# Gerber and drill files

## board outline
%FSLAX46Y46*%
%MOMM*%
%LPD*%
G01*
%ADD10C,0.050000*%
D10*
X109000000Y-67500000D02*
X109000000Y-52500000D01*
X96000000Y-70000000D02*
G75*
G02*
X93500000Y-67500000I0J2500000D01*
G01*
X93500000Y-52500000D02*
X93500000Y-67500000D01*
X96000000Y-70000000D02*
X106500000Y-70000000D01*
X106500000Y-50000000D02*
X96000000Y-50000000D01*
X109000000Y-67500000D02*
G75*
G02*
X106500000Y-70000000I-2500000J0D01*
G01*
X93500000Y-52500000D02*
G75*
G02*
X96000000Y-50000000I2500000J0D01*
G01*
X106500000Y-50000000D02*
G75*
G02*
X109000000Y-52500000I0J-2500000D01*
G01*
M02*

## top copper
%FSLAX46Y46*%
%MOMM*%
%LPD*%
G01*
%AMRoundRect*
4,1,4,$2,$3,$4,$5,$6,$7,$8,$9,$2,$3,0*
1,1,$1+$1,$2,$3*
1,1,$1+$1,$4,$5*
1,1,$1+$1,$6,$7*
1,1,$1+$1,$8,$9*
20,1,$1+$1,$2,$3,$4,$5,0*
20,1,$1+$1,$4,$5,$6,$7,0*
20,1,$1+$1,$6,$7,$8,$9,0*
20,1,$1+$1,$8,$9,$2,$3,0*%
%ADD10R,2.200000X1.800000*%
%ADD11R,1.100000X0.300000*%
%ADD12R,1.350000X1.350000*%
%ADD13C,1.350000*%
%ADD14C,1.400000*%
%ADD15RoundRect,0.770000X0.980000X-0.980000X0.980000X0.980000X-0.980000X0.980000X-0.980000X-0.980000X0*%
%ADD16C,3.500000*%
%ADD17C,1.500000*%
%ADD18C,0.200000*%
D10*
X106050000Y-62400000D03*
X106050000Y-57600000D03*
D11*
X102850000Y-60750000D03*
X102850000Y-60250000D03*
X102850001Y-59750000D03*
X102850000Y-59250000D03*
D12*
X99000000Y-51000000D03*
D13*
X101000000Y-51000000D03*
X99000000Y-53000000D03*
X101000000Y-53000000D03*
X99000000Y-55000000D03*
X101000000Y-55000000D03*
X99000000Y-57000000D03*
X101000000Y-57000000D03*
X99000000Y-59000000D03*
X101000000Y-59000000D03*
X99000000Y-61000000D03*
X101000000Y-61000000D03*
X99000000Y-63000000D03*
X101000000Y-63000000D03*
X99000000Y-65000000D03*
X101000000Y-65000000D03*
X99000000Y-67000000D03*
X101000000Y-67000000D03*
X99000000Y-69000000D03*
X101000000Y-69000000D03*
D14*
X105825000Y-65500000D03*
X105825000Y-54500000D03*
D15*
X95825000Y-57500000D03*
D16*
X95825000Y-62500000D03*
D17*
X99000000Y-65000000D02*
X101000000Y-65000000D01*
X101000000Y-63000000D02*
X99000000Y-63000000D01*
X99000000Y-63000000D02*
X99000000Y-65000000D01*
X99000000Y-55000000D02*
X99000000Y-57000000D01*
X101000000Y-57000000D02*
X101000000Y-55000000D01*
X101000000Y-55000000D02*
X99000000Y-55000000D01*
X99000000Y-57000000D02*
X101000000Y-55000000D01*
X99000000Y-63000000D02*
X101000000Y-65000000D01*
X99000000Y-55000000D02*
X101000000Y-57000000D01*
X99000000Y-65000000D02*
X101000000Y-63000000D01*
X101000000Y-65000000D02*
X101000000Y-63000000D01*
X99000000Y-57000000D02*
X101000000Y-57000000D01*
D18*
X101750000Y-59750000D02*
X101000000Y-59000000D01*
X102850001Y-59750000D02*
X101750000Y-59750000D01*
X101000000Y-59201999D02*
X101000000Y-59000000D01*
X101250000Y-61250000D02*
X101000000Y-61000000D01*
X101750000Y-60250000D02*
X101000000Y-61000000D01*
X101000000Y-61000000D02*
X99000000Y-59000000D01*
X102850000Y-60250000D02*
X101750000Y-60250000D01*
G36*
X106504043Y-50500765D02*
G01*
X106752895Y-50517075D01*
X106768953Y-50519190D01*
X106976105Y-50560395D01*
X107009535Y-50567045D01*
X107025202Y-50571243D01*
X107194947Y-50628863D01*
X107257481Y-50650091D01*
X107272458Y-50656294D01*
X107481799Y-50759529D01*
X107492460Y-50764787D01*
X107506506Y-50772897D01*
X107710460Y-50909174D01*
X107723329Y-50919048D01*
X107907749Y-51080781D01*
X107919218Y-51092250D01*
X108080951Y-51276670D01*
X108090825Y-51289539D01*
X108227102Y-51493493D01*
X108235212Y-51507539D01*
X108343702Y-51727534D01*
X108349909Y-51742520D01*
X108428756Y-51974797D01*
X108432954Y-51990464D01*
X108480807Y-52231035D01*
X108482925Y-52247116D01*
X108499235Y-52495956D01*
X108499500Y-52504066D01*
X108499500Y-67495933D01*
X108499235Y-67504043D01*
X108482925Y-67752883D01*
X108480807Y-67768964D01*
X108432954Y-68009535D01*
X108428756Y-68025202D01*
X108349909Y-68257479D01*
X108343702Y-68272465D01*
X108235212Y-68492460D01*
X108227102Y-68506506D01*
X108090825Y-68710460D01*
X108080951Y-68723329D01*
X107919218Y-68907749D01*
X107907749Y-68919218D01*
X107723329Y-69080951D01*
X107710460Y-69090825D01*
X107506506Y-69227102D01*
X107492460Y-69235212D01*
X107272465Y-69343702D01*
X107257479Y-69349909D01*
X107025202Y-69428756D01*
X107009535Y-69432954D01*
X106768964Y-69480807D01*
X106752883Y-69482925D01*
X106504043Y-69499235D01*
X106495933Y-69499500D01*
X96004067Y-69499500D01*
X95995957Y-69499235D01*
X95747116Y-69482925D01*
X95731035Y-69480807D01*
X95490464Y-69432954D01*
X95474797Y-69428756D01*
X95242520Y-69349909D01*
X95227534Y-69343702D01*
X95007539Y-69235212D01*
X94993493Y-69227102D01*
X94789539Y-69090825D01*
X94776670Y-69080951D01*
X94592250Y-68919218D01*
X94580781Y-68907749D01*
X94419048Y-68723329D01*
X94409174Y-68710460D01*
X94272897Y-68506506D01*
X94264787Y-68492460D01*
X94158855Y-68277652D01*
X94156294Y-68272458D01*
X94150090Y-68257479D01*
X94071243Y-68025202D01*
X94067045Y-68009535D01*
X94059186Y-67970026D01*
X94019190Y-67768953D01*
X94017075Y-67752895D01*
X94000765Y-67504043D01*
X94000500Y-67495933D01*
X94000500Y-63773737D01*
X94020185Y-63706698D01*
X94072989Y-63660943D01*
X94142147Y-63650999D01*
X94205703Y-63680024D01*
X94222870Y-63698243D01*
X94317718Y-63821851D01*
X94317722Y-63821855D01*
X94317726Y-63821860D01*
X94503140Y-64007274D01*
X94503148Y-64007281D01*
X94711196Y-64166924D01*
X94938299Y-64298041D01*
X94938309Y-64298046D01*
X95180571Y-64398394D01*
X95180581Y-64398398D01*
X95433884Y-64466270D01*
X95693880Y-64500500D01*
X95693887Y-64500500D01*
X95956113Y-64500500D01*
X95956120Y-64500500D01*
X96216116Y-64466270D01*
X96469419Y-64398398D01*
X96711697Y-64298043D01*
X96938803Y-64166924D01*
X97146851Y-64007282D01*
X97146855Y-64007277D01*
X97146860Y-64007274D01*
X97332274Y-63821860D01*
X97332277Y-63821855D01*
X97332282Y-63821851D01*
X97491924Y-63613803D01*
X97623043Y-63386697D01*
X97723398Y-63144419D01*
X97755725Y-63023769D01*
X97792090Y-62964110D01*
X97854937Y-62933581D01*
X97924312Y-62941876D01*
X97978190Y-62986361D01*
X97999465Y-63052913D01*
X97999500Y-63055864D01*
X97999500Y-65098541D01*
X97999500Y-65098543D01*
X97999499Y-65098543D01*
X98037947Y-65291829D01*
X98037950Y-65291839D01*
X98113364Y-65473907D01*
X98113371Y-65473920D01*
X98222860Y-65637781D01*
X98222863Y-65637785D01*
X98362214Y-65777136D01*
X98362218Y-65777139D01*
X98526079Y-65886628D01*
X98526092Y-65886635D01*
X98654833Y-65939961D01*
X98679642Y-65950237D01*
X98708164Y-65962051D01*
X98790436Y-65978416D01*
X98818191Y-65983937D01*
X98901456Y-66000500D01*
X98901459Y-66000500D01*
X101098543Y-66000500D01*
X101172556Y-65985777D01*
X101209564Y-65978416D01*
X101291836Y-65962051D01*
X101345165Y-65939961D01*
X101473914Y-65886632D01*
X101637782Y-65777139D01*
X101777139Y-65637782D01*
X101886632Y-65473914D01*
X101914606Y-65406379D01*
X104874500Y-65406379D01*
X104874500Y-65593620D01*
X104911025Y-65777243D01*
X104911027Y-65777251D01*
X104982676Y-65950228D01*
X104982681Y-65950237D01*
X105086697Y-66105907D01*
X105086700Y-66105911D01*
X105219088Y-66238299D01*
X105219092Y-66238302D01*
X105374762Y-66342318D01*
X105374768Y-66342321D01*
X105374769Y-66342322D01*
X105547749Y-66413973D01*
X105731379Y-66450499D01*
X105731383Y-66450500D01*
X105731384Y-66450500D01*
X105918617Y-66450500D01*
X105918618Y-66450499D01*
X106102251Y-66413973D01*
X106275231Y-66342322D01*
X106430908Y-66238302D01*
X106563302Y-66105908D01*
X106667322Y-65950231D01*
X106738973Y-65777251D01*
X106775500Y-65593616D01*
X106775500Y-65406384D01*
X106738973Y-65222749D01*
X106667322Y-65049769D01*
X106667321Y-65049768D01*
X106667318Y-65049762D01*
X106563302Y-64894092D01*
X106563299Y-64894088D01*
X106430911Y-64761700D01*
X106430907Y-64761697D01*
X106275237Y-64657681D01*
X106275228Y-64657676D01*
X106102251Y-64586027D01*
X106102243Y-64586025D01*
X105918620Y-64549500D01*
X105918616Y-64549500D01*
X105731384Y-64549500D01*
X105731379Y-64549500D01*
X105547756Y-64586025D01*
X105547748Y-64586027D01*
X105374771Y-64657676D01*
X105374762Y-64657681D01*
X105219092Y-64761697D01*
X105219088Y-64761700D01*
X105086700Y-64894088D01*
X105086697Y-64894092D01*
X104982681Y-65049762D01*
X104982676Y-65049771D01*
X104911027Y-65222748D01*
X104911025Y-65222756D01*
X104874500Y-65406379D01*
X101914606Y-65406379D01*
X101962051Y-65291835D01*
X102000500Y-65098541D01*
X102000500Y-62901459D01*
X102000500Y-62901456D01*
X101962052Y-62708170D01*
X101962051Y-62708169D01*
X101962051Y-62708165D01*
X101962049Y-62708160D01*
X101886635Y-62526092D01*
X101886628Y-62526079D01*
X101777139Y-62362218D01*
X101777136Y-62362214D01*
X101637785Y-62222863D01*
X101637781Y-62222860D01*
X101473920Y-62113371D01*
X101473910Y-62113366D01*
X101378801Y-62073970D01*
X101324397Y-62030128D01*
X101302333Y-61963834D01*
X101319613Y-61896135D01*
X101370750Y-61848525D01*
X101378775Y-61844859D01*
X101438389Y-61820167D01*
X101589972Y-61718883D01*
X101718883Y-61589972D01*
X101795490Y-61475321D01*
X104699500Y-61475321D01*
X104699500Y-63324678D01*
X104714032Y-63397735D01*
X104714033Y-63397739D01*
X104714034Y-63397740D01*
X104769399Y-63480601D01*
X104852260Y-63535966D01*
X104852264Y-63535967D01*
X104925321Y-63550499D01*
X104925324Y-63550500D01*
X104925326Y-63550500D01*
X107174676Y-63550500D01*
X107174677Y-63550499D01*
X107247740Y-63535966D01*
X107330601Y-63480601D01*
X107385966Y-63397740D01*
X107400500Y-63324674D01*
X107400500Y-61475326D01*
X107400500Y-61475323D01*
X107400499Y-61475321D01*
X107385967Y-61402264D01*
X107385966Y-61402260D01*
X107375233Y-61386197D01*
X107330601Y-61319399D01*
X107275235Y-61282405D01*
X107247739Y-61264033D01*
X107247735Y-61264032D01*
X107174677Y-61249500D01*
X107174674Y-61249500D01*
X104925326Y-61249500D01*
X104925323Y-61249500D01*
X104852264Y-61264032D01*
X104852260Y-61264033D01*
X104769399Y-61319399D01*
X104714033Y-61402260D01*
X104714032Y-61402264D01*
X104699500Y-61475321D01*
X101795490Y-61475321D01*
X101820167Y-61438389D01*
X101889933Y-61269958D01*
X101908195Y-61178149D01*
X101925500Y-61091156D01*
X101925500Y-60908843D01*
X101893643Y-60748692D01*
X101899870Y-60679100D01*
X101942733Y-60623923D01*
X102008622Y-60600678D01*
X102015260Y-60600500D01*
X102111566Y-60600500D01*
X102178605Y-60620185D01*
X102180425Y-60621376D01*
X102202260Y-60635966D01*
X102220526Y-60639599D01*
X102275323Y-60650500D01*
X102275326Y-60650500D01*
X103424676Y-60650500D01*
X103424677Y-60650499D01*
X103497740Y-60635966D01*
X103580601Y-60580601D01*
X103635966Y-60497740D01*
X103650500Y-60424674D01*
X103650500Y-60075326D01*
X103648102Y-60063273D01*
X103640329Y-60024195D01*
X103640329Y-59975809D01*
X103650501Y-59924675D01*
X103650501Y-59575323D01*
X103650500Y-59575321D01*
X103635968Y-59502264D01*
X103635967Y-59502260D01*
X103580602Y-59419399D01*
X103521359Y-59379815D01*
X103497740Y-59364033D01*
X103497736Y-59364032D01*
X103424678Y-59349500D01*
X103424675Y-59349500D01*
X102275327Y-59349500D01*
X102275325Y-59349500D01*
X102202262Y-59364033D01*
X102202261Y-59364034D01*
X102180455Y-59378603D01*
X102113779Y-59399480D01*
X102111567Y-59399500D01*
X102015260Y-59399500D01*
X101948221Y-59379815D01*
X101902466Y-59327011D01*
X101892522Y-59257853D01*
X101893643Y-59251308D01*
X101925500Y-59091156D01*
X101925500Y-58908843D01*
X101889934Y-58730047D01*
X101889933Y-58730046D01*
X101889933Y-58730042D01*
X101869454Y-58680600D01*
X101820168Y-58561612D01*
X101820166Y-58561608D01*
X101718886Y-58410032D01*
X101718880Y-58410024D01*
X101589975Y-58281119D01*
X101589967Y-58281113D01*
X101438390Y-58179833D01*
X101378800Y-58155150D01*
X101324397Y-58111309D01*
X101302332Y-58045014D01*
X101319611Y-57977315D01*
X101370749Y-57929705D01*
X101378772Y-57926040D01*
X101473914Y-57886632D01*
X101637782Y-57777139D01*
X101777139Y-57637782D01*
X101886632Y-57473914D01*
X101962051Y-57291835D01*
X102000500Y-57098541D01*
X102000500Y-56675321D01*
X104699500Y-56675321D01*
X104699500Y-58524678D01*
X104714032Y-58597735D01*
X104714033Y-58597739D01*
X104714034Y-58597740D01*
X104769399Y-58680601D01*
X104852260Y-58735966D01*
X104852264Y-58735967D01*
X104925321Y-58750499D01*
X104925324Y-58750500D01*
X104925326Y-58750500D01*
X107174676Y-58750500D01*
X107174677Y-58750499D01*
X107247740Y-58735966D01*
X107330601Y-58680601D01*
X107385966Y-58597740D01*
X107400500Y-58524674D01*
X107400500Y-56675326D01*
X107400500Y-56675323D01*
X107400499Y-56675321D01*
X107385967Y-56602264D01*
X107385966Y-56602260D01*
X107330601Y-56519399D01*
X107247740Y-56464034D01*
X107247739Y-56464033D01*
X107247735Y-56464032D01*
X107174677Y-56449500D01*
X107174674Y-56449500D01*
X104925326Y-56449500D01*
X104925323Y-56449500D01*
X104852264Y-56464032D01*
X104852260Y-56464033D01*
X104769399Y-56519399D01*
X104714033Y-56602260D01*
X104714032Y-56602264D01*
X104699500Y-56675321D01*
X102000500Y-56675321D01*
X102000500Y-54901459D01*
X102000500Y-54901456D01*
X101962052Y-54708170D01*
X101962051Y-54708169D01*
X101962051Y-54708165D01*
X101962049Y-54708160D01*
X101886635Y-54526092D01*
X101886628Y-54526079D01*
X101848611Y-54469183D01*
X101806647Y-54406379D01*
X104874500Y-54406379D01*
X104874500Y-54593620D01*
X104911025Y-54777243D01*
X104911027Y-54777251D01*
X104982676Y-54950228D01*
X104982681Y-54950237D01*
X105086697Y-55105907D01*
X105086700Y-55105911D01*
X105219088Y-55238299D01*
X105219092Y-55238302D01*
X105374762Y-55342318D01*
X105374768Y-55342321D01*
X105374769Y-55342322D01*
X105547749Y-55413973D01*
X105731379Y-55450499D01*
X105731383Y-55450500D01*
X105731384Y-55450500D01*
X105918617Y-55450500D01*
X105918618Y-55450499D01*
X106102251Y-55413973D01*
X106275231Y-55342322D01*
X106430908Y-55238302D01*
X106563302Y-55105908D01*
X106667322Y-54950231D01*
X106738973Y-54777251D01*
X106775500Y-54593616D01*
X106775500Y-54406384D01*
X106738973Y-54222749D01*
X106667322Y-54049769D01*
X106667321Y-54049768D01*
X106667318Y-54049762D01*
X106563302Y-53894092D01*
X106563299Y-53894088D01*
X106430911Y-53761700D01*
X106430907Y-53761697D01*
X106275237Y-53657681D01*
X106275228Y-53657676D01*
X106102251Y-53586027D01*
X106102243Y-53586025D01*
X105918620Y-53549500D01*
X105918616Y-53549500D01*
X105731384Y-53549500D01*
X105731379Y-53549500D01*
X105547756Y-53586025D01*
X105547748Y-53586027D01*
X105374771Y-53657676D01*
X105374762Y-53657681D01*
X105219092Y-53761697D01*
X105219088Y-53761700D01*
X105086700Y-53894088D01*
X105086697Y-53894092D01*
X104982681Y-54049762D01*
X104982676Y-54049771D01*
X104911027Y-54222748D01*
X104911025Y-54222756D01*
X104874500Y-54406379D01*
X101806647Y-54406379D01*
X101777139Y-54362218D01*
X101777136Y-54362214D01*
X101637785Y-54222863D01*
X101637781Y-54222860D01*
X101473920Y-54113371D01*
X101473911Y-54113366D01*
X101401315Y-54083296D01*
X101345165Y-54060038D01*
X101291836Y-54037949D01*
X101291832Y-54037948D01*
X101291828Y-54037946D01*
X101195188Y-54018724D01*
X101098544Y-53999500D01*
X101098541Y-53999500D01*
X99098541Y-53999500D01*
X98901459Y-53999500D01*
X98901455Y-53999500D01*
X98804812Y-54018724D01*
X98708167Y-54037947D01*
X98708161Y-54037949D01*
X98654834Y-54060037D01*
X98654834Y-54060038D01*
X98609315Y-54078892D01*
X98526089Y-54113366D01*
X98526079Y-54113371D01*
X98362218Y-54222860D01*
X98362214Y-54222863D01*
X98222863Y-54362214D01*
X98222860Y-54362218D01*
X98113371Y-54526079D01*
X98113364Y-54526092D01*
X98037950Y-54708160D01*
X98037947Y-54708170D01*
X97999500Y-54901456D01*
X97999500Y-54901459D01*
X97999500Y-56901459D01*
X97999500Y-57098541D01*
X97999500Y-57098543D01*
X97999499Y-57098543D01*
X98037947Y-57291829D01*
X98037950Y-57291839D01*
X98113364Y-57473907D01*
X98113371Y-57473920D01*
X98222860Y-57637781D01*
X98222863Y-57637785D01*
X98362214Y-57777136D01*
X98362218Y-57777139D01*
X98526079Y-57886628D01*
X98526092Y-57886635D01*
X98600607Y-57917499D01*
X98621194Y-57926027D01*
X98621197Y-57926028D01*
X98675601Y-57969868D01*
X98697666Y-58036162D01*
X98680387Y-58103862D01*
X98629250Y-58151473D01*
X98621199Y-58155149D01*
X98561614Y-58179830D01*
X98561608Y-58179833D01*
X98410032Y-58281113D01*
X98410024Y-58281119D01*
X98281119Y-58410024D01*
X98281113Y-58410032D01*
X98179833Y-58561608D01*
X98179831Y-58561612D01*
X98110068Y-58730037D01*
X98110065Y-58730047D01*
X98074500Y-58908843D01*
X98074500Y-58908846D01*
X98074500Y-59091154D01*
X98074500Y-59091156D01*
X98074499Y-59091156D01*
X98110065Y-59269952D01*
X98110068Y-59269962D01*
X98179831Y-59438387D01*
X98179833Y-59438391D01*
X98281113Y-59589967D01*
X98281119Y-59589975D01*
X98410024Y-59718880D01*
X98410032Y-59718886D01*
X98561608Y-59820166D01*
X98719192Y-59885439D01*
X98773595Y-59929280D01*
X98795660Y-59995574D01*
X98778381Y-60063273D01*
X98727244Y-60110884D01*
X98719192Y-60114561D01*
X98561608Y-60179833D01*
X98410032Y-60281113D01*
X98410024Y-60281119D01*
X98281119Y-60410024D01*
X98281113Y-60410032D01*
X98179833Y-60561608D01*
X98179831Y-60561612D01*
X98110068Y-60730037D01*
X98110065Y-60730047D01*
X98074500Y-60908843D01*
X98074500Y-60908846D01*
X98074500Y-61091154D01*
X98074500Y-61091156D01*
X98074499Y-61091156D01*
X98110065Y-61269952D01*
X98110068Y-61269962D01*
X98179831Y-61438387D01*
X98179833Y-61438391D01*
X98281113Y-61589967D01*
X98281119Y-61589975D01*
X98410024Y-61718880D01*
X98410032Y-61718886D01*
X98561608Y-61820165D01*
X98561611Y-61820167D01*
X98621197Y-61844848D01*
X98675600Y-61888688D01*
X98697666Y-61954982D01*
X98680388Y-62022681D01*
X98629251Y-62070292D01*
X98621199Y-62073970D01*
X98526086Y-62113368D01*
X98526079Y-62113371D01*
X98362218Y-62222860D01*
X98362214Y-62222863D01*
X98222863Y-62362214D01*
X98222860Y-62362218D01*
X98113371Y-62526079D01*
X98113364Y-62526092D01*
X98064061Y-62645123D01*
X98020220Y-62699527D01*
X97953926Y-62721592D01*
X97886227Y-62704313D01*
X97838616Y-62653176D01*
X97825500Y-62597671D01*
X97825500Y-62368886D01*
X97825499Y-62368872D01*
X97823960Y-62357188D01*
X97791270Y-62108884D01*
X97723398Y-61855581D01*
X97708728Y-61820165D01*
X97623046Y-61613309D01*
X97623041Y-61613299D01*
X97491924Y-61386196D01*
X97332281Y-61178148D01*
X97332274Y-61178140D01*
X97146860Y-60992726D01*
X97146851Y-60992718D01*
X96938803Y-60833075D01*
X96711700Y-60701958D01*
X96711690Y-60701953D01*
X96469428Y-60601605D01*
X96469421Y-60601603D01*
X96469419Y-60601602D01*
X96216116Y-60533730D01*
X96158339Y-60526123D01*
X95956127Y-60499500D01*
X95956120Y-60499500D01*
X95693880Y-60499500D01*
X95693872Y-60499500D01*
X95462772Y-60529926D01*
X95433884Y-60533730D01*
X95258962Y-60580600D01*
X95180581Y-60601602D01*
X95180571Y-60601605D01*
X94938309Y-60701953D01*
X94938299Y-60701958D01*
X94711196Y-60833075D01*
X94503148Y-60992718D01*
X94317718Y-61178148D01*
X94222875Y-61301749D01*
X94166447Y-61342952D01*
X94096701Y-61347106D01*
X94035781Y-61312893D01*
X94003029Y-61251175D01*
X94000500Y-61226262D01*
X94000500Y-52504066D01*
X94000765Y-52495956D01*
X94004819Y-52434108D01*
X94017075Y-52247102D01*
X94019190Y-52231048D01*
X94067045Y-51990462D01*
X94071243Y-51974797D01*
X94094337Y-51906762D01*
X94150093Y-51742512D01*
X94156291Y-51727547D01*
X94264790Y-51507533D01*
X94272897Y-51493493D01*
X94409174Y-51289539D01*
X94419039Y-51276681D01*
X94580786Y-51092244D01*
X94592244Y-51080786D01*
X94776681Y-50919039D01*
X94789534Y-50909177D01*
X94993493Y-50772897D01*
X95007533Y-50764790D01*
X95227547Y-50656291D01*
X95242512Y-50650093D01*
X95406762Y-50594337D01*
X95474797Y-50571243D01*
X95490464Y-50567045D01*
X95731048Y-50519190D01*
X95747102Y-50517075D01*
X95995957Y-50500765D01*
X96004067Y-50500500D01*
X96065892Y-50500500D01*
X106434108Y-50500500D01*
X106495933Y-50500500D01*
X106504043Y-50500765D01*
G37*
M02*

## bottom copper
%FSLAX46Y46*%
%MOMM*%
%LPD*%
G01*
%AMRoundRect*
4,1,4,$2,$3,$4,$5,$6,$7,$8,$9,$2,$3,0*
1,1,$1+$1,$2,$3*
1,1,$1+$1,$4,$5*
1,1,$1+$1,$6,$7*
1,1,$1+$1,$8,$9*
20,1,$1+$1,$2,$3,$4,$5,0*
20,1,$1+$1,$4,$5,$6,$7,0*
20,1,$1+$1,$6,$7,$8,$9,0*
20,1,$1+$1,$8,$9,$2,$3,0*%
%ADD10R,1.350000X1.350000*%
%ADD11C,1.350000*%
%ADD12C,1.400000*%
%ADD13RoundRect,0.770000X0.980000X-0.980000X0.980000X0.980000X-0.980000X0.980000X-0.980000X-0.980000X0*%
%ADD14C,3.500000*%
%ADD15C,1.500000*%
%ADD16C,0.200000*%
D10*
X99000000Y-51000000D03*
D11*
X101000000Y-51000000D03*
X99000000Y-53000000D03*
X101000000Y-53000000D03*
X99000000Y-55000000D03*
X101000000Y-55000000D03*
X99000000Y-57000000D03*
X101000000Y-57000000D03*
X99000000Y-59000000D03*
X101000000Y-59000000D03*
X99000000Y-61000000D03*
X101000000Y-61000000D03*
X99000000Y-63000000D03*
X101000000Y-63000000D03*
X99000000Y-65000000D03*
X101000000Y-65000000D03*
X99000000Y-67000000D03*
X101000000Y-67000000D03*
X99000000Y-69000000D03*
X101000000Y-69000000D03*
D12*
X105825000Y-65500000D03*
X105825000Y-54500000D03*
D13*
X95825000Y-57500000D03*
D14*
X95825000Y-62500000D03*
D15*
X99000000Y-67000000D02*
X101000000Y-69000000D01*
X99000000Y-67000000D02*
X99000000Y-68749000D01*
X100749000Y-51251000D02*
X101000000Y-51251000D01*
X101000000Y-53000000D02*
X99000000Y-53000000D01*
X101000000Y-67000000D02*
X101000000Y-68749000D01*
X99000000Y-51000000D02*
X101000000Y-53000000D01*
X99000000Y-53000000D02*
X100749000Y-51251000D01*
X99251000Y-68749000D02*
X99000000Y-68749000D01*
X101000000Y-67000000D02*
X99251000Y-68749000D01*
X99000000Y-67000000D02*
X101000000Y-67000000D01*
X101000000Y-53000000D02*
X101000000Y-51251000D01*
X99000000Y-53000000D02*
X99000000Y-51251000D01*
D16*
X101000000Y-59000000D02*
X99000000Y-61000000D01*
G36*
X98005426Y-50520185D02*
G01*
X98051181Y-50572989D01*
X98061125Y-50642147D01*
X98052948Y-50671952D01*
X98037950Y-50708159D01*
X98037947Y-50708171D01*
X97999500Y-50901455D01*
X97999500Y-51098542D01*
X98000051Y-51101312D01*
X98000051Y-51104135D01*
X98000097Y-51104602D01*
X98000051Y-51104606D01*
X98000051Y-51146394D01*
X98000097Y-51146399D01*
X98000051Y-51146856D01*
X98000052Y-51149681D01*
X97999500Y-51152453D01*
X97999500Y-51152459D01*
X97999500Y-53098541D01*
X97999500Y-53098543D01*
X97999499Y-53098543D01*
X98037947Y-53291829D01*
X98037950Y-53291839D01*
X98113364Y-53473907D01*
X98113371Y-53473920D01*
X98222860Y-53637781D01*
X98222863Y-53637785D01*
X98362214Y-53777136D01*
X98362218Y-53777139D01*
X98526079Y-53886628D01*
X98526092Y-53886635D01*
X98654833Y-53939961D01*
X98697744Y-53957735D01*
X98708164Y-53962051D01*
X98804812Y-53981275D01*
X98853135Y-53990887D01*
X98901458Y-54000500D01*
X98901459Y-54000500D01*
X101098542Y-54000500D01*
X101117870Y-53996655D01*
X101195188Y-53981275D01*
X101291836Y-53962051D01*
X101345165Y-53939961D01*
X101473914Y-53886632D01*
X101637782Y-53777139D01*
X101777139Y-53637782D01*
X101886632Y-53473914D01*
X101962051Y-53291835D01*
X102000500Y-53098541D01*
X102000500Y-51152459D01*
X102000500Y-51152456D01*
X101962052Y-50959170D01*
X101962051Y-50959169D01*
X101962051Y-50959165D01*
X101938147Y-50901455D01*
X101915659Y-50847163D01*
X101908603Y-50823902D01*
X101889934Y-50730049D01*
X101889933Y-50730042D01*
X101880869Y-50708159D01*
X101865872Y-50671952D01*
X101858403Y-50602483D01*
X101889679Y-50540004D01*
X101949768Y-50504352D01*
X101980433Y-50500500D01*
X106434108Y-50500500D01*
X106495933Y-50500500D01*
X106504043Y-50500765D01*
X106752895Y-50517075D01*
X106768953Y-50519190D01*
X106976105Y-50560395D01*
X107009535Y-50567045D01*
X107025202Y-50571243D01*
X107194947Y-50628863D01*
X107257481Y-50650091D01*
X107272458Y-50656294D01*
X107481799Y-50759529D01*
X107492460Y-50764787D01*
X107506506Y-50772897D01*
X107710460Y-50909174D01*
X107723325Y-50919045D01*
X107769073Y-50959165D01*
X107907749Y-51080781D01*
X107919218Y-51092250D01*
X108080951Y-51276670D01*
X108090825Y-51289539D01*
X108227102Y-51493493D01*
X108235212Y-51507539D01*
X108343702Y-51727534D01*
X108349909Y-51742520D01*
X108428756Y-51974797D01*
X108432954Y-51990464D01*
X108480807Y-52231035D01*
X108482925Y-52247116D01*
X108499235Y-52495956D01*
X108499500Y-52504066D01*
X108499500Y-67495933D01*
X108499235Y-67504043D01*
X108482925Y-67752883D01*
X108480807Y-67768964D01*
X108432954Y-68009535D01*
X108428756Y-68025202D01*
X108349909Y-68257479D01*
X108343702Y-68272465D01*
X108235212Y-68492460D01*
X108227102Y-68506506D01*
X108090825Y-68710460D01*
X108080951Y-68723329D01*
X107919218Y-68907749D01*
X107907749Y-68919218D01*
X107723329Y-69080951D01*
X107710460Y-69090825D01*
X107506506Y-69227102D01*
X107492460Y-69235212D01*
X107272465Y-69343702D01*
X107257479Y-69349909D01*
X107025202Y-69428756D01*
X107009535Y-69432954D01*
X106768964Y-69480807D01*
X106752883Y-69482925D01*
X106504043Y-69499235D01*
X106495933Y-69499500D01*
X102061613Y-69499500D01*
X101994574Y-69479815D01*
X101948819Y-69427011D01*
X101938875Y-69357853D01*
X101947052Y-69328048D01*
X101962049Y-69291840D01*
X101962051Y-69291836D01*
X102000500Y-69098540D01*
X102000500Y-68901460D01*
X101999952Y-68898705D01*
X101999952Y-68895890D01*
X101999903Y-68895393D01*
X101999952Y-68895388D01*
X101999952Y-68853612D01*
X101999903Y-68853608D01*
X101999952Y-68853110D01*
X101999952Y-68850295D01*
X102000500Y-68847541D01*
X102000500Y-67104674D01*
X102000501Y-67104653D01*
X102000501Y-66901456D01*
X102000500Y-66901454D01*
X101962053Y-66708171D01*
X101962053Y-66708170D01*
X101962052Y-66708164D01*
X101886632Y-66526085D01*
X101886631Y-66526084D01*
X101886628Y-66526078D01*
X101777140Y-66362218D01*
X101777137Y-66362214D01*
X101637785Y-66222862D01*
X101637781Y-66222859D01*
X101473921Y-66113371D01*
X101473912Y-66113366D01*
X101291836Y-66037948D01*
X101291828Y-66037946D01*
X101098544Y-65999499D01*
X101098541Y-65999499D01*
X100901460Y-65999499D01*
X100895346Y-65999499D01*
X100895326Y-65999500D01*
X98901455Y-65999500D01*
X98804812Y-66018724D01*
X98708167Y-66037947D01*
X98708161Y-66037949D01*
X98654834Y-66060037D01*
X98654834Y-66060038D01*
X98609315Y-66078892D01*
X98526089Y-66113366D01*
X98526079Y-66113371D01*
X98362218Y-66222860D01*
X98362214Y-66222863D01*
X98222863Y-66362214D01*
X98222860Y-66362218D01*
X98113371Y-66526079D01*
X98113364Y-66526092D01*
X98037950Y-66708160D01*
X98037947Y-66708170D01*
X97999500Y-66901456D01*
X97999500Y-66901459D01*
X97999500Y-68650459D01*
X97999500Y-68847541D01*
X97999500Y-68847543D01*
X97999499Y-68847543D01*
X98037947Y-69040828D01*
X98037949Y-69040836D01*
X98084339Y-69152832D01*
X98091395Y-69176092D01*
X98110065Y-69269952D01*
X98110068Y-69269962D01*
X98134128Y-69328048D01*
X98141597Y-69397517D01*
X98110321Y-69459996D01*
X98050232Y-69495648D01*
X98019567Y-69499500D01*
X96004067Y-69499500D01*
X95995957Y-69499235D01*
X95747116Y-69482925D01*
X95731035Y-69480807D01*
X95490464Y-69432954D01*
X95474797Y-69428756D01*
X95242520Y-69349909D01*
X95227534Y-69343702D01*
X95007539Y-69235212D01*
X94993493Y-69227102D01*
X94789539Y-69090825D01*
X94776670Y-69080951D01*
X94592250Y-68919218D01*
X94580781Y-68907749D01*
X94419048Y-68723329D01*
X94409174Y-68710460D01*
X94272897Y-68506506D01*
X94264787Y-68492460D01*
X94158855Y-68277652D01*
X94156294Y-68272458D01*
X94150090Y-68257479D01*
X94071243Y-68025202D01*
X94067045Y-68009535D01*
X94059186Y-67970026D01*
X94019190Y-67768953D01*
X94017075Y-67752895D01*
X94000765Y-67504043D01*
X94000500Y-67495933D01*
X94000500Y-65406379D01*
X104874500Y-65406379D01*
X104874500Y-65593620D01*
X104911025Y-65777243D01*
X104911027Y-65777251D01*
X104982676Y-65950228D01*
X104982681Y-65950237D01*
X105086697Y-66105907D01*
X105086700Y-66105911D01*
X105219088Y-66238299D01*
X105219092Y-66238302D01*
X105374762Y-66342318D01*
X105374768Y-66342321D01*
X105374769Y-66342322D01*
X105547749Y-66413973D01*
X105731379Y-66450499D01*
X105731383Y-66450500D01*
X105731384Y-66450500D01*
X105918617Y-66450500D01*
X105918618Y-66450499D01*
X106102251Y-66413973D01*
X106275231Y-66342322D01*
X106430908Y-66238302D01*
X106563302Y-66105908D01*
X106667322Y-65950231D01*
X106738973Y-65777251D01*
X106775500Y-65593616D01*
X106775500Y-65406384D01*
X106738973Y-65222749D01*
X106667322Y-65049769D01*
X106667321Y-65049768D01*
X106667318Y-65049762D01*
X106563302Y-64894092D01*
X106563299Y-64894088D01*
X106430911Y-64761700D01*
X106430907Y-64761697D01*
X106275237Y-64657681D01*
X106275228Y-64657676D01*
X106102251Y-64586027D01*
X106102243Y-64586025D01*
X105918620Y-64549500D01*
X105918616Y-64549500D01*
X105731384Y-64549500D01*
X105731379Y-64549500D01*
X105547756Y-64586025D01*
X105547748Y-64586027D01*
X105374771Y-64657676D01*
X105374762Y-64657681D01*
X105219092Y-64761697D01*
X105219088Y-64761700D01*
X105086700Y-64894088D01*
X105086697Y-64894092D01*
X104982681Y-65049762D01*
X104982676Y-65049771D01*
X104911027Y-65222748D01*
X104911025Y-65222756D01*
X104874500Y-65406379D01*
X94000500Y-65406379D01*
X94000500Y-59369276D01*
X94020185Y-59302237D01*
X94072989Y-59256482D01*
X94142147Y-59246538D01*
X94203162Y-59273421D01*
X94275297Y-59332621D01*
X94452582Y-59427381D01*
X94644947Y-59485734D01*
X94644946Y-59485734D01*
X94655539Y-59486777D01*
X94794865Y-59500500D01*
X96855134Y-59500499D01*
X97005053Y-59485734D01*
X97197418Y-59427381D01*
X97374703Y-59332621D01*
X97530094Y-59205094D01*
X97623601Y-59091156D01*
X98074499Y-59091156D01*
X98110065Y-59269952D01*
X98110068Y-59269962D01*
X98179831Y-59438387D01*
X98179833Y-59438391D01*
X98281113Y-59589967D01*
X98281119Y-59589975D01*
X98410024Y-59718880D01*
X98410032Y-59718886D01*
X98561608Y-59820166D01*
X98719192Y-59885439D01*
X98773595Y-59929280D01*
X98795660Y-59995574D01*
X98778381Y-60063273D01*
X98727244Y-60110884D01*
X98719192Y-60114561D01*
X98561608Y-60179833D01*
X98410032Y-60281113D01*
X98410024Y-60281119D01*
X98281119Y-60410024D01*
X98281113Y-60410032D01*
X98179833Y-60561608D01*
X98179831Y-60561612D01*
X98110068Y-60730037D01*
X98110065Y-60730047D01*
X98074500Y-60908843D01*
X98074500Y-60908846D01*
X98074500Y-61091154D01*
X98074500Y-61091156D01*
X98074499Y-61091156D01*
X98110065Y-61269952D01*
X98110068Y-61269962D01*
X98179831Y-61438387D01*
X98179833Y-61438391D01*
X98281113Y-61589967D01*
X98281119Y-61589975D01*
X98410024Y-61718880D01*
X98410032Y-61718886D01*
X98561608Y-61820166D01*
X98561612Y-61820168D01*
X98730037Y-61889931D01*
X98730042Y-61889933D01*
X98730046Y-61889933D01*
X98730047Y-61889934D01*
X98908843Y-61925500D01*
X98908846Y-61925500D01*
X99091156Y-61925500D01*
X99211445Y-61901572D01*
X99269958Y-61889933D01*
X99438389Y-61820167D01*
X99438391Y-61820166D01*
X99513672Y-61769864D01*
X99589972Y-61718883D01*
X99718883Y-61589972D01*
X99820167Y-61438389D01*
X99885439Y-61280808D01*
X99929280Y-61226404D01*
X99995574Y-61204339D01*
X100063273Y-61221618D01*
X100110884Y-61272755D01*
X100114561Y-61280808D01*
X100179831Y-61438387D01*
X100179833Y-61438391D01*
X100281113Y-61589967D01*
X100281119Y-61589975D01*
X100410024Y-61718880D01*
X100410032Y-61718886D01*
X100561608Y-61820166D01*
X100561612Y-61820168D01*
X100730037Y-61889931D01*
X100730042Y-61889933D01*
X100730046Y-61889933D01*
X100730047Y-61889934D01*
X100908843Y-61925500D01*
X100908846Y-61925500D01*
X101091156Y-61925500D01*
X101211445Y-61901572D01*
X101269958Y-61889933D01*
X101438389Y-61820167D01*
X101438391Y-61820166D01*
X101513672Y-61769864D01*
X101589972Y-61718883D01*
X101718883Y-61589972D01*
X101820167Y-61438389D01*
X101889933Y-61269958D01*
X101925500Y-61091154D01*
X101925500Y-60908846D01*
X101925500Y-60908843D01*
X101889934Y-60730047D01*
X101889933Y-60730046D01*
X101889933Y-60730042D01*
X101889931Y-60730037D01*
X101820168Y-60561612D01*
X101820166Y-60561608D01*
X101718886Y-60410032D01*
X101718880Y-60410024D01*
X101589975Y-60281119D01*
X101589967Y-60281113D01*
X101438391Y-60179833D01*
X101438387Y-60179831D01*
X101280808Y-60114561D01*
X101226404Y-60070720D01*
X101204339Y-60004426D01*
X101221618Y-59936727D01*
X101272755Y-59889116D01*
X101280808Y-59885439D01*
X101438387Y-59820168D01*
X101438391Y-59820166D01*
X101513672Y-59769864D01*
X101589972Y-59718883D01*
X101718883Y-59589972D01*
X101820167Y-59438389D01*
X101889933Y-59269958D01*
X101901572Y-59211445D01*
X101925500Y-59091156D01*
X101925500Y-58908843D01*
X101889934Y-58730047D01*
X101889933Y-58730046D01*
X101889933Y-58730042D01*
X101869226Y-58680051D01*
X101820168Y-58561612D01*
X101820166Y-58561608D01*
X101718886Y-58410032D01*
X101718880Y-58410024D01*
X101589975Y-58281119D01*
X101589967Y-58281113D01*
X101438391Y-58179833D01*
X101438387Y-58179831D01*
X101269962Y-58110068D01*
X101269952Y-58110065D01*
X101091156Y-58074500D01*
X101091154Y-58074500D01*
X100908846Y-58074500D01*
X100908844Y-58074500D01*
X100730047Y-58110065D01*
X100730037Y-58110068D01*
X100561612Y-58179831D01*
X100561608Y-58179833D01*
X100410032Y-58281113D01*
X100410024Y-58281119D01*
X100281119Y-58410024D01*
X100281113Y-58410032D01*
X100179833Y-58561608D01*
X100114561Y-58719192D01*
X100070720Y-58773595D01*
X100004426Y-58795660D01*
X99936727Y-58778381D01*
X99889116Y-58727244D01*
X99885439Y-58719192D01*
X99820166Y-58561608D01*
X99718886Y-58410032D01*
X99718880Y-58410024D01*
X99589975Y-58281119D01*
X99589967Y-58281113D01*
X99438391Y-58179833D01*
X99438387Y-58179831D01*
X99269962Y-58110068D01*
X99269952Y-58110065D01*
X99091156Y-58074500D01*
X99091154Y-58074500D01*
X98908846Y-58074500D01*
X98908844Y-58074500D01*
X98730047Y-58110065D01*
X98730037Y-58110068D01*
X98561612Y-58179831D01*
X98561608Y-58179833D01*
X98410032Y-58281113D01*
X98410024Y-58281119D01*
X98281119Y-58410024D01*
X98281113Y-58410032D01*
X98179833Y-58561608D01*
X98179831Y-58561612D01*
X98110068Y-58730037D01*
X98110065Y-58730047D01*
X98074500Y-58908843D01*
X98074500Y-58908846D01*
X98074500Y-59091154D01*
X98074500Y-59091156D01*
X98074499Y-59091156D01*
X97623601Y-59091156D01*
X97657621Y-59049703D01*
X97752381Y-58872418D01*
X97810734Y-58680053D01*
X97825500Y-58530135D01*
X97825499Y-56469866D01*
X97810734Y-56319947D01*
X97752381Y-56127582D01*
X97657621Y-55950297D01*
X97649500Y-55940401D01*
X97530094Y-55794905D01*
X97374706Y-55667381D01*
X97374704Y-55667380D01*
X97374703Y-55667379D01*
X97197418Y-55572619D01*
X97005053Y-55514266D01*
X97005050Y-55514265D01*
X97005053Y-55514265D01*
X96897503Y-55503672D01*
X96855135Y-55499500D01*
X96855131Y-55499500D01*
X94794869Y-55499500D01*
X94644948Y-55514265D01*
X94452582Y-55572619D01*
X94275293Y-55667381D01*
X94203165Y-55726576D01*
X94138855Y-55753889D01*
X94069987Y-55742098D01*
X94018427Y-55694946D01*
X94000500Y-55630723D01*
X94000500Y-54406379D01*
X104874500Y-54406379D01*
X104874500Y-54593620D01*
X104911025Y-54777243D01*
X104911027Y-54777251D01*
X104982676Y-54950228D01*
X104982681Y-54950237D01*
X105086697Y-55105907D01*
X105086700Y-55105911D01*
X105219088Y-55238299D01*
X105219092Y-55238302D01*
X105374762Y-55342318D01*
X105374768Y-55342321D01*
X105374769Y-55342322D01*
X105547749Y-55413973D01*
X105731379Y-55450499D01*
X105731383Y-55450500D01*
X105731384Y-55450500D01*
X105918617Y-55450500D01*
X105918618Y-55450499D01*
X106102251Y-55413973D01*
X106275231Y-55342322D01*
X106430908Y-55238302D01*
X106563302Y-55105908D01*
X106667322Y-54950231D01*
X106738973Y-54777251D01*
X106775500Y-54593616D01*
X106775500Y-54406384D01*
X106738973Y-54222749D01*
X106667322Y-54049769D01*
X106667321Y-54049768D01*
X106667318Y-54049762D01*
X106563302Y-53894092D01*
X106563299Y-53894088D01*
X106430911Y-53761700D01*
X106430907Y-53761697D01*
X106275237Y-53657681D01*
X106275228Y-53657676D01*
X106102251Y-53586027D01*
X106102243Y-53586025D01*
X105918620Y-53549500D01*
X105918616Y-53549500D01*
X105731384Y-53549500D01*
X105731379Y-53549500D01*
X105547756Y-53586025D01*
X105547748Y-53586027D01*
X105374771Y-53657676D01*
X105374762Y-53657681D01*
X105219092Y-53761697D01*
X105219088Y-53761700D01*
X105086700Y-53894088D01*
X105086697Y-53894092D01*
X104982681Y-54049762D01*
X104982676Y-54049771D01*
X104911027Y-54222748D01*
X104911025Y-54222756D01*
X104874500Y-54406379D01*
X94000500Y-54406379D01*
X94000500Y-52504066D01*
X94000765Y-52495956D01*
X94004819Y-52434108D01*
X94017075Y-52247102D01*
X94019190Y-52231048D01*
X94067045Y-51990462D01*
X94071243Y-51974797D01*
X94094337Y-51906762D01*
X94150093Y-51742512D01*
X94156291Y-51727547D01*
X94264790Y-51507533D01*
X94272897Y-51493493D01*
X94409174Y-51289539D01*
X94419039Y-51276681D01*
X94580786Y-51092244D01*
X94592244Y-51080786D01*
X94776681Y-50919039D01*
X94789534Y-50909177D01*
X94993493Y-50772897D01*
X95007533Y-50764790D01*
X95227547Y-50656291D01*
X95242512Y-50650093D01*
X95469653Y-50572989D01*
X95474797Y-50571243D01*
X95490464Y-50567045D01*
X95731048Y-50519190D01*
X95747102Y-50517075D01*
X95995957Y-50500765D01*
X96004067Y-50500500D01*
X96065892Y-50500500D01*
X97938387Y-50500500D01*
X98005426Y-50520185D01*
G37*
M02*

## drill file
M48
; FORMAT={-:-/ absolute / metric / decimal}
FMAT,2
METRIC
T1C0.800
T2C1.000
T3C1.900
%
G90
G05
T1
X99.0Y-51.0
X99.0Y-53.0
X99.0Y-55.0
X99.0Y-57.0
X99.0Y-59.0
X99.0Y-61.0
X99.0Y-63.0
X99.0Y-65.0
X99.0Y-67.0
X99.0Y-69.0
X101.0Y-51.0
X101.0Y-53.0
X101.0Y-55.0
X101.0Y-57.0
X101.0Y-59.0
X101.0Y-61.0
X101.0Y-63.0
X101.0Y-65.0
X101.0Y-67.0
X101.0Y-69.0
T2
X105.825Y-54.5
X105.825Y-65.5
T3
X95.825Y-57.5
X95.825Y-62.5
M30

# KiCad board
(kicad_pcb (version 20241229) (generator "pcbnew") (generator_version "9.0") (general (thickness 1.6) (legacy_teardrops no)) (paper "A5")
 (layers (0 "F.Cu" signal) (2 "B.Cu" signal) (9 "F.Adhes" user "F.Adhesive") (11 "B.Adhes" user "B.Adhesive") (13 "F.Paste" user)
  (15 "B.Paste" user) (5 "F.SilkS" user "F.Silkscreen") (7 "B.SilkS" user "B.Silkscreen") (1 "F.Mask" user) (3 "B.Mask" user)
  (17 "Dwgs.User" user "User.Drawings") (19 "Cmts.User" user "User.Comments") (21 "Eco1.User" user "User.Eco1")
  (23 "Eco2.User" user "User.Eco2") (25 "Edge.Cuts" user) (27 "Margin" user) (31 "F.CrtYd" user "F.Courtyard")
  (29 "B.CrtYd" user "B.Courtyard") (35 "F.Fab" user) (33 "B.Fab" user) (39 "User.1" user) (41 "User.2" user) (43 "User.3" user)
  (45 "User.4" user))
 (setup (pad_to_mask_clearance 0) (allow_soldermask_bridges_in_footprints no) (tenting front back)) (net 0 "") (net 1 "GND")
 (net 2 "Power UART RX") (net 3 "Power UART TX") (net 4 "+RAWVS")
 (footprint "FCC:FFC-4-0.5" (layer "F.Cu") (at 103.5 60 90)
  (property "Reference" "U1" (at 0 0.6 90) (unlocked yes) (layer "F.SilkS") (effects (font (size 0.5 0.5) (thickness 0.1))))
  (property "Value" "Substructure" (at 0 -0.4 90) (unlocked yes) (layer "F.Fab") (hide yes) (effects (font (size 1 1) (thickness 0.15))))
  (pad "" smd rect (at -2.4 2.55 90) (size 1.8 2.2) (layers "F.Cu" "F.Mask" "F.Paste") (thermal_bridge_angle 45))
  (pad "" smd rect (at 2.4 2.55 90) (size 1.8 2.2) (layers "F.Cu" "F.Mask" "F.Paste") (thermal_bridge_angle 45))
  (pad "1" smd rect (at -0.75 -0.65 90) (size 0.3 1.1) (layers "F.Cu" "F.Mask" "F.Paste") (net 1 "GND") (thermal_bridge_angle 45))
  (pad "2" smd rect (at -0.25 -0.65 90) (size 0.3 1.1) (layers "F.Cu" "F.Mask" "F.Paste") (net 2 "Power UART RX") (thermal_bridge_angle 45))
  (pad "3" smd rect (at 0.25 -0.649999 90) (size 0.3 1.1) (layers "F.Cu" "F.Mask" "F.Paste") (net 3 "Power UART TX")
   (thermal_bridge_angle 45))
  (pad "4" smd rect (at 0.75 -0.65 90) (size 0.3 1.1) (layers "F.Cu" "F.Mask" "F.Paste") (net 1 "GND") (thermal_bridge_angle 45)))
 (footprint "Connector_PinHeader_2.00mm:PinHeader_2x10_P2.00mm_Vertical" (layer "F.Cu") (at 99 51)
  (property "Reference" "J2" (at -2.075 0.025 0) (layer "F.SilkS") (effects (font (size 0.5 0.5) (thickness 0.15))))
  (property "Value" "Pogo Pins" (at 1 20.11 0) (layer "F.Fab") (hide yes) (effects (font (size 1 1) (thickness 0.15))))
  (pad "1" thru_hole rect (at 0 0) (size 1.35 1.35) (drill 0.8) (layers "*.Cu" "*.Mask") (remove_unused_layers no) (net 1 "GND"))
  (pad "2" thru_hole circle (at 2 0) (size 1.35 1.35) (drill 0.8) (layers "*.Cu" "*.Mask") (remove_unused_layers no) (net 1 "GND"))
  (pad "3" thru_hole circle (at 0 2) (size 1.35 1.35) (drill 0.8) (layers "*.Cu" "*.Mask") (remove_unused_layers no) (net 1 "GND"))
  (pad "4" thru_hole circle (at 2 2) (size 1.35 1.35) (drill 0.8) (layers "*.Cu" "*.Mask") (remove_unused_layers no) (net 1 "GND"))
  (pad "5" thru_hole circle (at 0 4) (size 1.35 1.35) (drill 0.8) (layers "*.Cu" "*.Mask") (remove_unused_layers no) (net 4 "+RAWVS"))
  (pad "6" thru_hole circle (at 2 4) (size 1.35 1.35) (drill 0.8) (layers "*.Cu" "*.Mask") (remove_unused_layers no) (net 4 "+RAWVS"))
  (pad "7" thru_hole circle (at 0 6) (size 1.35 1.35) (drill 0.8) (layers "*.Cu" "*.Mask") (remove_unused_layers no) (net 4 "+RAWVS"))
  (pad "8" thru_hole circle (at 2 6) (size 1.35 1.35) (drill 0.8) (layers "*.Cu" "*.Mask") (remove_unused_layers no) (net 4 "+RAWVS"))
  (pad "9" thru_hole circle (at 0 8) (size 1.35 1.35) (drill 0.8) (layers "*.Cu" "*.Mask") (remove_unused_layers no) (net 2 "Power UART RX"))
  (pad "10" thru_hole circle (at 2 8) (size 1.35 1.35) (drill 0.8) (layers "*.Cu" "*.Mask") (remove_unused_layers no)
   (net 3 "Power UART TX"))
  (pad "11" thru_hole circle (at 0 10) (size 1.35 1.35) (drill 0.8) (layers "*.Cu" "*.Mask") (remove_unused_layers no)
   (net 3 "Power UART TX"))
  (pad "12" thru_hole circle (at 2 10) (size 1.35 1.35) (drill 0.8) (layers "*.Cu" "*.Mask") (remove_unused_layers no)
   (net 2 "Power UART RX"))
  (pad "13" thru_hole circle (at 0 12) (size 1.35 1.35) (drill 0.8) (layers "*.Cu" "*.Mask") (remove_unused_layers no) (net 4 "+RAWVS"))
  (pad "14" thru_hole circle (at 2 12) (size 1.35 1.35) (drill 0.8) (layers "*.Cu" "*.Mask") (remove_unused_layers no) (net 4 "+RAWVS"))
  (pad "15" thru_hole circle (at 0 14) (size 1.35 1.35) (drill 0.8) (layers "*.Cu" "*.Mask") (remove_unused_layers no) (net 4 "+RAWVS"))
  (pad "16" thru_hole circle (at 2 14) (size 1.35 1.35) (drill 0.8) (layers "*.Cu" "*.Mask") (remove_unused_layers no) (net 4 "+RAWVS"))
  (pad "17" thru_hole circle (at 0 16) (size 1.35 1.35) (drill 0.8) (layers "*.Cu" "*.Mask") (remove_unused_layers no) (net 1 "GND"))
  (pad "18" thru_hole circle (at 2 16) (size 1.35 1.35) (drill 0.8) (layers "*.Cu" "*.Mask") (remove_unused_layers no) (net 1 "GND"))
  (pad "19" thru_hole circle (at 0 18) (size 1.35 1.35) (drill 0.8) (layers "*.Cu" "*.Mask") (remove_unused_layers no) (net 1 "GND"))
  (pad "20" thru_hole circle (at 2 18) (size 1.35 1.35) (drill 0.8) (layers "*.Cu" "*.Mask") (remove_unused_layers no) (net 1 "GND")))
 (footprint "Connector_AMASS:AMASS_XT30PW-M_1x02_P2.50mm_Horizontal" (layer "B.Cu") (at 95.825 57.5 90)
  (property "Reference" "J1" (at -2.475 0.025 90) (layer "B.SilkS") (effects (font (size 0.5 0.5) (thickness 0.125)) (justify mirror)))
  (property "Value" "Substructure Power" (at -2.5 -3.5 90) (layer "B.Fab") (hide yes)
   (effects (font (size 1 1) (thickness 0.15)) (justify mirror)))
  (pad "" thru_hole circle (at -8 10 90) (size 1.4 1.4) (drill 1) (layers "*.Cu" "*.Mask") (remove_unused_layers no))
  (pad "" thru_hole circle (at 3 10 90) (size 1.4 1.4) (drill 1) (layers "*.Cu" "*.Mask") (remove_unused_layers no))
  (pad "1" thru_hole roundrect (at 0 0 90) (size 3.5 3.5) (drill 1.9) (layers "*.Cu" "*.Mask") (remove_unused_layers no)
   (roundrect_rratio 0.22) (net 1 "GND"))
  (pad "2" thru_hole circle (at -5 0 90) (size 3.5 3.5) (drill 1.9) (layers "*.Cu" "*.Mask") (remove_unused_layers no) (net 4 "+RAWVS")))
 (gr_line (start 109 67.5) (end 109 52.5) (stroke (width 0.05) (type default)) (layer "Edge.Cuts"))
 (gr_arc (start 96 70) (mid 94.232233 69.267767) (end 93.5 67.5) (stroke (width 0.05) (type default)) (layer "Edge.Cuts"))
 (gr_line (start 93.5 52.5) (end 93.5 67.5) (stroke (width 0.05) (type default)) (layer "Edge.Cuts"))
 (gr_line (start 96 70) (end 106.5 70) (stroke (width 0.05) (type default)) (layer "Edge.Cuts"))
 (gr_line (start 106.5 50) (end 96 50) (stroke (width 0.05) (type default)) (layer "Edge.Cuts"))
 (gr_arc (start 109 67.5) (mid 108.267767 69.267767) (end 106.5 70) (stroke (width 0.05) (type default)) (layer "Edge.Cuts"))
 (gr_arc (start 93.5 52.5) (mid 94.232233 50.732233) (end 96 50) (stroke (width 0.05) (type default)) (layer "Edge.Cuts"))
 (gr_arc (start 106.5 50) (mid 108.267767 50.732233) (end 109 52.5) (stroke (width 0.05) (type default)) (layer "Edge.Cuts"))
 (segment (start 99 65) (end 101 65) (width 1.5) (layer "F.Cu") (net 4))
 (segment (start 101 63) (end 99 63) (width 1.5) (layer "F.Cu") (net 4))
 (segment (start 99 63) (end 99 65) (width 1.5) (layer "F.Cu") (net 4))
 (segment (start 99 55) (end 99 57) (width 1.5) (layer "F.Cu") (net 4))
 (segment (start 101 57) (end 101 55) (width 1.5) (layer "F.Cu") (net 4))
 (segment (start 101 55) (end 99 55) (width 1.5) (layer "F.Cu") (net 4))
 (segment (start 99 57) (end 101 55) (width 1.5) (layer "F.Cu") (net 4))
 (segment (start 99 63) (end 101 65) (width 1.5) (layer "F.Cu") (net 4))
 (segment (start 99 55) (end 101 57) (width 1.5) (layer "F.Cu") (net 4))
 (segment (start 99 65) (end 101 63) (width 1.5) (layer "F.Cu") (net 4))
 (segment (start 101 65) (end 101 63) (width 1.5) (layer "F.Cu") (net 4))
 (segment (start 99 57) (end 101 57) (width 1.5) (layer "F.Cu") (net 4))
 (segment (start 99 67) (end 101 69) (width 1.5) (layer "B.Cu") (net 1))
 (segment (start 99 67) (end 99 68.749) (width 1.5) (layer "B.Cu") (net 1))
 (segment (start 100.749 51.251) (end 101 51.251) (width 1.5) (layer "B.Cu") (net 1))
 (segment (start 101 53) (end 99 53) (width 1.5) (layer "B.Cu") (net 1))
 (segment (start 101 67) (end 101 68.749) (width 1.5) (layer "B.Cu") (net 1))
 (segment (start 99 51) (end 101 53) (width 1.5) (layer "B.Cu") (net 1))
 (segment (start 99 53) (end 100.749 51.251) (width 1.5) (layer "B.Cu") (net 1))
 (segment (start 99.251 68.749) (end 99 68.749) (width 1.5) (layer "B.Cu") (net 1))
 (segment (start 101 67) (end 99.251 68.749) (width 1.5) (layer "B.Cu") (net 1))
 (segment (start 99 67) (end 101 67) (width 1.5) (layer "B.Cu") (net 1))
 (segment (start 101 53) (end 101 51.251) (width 1.5) (layer "B.Cu") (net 1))
 (segment (start 99 53) (end 99 51.251) (width 1.5) (layer "B.Cu") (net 1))
 (segment (start 101.75 59.75) (end 101 59) (width 0.2) (layer "F.Cu") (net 3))
 (segment (start 102.850001 59.75) (end 101.75 59.75) (width 0.2) (layer "F.Cu") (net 3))
 (segment (start 101 59.201999) (end 101 59) (width 0.2) (layer "F.Cu") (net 3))
 (segment (start 101 59) (end 99 61) (width 0.2) (layer "B.Cu") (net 3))
 (segment (start 101.25 61.25) (end 101 61) (width 0.2) (layer "F.Cu") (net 2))
 (segment (start 101.75 60.25) (end 101 61) (width 0.2) (layer "F.Cu") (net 2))
 (segment (start 101 61) (end 99 59) (width 0.2) (layer "F.Cu") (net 2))
 (segment (start 102.85 60.25) (end 101.75 60.25) (width 0.2) (layer "F.Cu") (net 2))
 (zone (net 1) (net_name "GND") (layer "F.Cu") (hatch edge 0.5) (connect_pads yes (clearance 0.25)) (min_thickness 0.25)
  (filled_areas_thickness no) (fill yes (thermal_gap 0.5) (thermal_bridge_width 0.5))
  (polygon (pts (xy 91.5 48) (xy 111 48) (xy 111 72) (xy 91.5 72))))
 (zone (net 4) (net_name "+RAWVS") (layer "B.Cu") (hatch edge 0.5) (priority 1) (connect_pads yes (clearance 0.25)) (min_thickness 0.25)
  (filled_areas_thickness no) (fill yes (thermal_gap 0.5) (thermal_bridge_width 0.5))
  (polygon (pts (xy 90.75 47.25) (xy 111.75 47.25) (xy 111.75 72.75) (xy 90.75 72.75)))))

